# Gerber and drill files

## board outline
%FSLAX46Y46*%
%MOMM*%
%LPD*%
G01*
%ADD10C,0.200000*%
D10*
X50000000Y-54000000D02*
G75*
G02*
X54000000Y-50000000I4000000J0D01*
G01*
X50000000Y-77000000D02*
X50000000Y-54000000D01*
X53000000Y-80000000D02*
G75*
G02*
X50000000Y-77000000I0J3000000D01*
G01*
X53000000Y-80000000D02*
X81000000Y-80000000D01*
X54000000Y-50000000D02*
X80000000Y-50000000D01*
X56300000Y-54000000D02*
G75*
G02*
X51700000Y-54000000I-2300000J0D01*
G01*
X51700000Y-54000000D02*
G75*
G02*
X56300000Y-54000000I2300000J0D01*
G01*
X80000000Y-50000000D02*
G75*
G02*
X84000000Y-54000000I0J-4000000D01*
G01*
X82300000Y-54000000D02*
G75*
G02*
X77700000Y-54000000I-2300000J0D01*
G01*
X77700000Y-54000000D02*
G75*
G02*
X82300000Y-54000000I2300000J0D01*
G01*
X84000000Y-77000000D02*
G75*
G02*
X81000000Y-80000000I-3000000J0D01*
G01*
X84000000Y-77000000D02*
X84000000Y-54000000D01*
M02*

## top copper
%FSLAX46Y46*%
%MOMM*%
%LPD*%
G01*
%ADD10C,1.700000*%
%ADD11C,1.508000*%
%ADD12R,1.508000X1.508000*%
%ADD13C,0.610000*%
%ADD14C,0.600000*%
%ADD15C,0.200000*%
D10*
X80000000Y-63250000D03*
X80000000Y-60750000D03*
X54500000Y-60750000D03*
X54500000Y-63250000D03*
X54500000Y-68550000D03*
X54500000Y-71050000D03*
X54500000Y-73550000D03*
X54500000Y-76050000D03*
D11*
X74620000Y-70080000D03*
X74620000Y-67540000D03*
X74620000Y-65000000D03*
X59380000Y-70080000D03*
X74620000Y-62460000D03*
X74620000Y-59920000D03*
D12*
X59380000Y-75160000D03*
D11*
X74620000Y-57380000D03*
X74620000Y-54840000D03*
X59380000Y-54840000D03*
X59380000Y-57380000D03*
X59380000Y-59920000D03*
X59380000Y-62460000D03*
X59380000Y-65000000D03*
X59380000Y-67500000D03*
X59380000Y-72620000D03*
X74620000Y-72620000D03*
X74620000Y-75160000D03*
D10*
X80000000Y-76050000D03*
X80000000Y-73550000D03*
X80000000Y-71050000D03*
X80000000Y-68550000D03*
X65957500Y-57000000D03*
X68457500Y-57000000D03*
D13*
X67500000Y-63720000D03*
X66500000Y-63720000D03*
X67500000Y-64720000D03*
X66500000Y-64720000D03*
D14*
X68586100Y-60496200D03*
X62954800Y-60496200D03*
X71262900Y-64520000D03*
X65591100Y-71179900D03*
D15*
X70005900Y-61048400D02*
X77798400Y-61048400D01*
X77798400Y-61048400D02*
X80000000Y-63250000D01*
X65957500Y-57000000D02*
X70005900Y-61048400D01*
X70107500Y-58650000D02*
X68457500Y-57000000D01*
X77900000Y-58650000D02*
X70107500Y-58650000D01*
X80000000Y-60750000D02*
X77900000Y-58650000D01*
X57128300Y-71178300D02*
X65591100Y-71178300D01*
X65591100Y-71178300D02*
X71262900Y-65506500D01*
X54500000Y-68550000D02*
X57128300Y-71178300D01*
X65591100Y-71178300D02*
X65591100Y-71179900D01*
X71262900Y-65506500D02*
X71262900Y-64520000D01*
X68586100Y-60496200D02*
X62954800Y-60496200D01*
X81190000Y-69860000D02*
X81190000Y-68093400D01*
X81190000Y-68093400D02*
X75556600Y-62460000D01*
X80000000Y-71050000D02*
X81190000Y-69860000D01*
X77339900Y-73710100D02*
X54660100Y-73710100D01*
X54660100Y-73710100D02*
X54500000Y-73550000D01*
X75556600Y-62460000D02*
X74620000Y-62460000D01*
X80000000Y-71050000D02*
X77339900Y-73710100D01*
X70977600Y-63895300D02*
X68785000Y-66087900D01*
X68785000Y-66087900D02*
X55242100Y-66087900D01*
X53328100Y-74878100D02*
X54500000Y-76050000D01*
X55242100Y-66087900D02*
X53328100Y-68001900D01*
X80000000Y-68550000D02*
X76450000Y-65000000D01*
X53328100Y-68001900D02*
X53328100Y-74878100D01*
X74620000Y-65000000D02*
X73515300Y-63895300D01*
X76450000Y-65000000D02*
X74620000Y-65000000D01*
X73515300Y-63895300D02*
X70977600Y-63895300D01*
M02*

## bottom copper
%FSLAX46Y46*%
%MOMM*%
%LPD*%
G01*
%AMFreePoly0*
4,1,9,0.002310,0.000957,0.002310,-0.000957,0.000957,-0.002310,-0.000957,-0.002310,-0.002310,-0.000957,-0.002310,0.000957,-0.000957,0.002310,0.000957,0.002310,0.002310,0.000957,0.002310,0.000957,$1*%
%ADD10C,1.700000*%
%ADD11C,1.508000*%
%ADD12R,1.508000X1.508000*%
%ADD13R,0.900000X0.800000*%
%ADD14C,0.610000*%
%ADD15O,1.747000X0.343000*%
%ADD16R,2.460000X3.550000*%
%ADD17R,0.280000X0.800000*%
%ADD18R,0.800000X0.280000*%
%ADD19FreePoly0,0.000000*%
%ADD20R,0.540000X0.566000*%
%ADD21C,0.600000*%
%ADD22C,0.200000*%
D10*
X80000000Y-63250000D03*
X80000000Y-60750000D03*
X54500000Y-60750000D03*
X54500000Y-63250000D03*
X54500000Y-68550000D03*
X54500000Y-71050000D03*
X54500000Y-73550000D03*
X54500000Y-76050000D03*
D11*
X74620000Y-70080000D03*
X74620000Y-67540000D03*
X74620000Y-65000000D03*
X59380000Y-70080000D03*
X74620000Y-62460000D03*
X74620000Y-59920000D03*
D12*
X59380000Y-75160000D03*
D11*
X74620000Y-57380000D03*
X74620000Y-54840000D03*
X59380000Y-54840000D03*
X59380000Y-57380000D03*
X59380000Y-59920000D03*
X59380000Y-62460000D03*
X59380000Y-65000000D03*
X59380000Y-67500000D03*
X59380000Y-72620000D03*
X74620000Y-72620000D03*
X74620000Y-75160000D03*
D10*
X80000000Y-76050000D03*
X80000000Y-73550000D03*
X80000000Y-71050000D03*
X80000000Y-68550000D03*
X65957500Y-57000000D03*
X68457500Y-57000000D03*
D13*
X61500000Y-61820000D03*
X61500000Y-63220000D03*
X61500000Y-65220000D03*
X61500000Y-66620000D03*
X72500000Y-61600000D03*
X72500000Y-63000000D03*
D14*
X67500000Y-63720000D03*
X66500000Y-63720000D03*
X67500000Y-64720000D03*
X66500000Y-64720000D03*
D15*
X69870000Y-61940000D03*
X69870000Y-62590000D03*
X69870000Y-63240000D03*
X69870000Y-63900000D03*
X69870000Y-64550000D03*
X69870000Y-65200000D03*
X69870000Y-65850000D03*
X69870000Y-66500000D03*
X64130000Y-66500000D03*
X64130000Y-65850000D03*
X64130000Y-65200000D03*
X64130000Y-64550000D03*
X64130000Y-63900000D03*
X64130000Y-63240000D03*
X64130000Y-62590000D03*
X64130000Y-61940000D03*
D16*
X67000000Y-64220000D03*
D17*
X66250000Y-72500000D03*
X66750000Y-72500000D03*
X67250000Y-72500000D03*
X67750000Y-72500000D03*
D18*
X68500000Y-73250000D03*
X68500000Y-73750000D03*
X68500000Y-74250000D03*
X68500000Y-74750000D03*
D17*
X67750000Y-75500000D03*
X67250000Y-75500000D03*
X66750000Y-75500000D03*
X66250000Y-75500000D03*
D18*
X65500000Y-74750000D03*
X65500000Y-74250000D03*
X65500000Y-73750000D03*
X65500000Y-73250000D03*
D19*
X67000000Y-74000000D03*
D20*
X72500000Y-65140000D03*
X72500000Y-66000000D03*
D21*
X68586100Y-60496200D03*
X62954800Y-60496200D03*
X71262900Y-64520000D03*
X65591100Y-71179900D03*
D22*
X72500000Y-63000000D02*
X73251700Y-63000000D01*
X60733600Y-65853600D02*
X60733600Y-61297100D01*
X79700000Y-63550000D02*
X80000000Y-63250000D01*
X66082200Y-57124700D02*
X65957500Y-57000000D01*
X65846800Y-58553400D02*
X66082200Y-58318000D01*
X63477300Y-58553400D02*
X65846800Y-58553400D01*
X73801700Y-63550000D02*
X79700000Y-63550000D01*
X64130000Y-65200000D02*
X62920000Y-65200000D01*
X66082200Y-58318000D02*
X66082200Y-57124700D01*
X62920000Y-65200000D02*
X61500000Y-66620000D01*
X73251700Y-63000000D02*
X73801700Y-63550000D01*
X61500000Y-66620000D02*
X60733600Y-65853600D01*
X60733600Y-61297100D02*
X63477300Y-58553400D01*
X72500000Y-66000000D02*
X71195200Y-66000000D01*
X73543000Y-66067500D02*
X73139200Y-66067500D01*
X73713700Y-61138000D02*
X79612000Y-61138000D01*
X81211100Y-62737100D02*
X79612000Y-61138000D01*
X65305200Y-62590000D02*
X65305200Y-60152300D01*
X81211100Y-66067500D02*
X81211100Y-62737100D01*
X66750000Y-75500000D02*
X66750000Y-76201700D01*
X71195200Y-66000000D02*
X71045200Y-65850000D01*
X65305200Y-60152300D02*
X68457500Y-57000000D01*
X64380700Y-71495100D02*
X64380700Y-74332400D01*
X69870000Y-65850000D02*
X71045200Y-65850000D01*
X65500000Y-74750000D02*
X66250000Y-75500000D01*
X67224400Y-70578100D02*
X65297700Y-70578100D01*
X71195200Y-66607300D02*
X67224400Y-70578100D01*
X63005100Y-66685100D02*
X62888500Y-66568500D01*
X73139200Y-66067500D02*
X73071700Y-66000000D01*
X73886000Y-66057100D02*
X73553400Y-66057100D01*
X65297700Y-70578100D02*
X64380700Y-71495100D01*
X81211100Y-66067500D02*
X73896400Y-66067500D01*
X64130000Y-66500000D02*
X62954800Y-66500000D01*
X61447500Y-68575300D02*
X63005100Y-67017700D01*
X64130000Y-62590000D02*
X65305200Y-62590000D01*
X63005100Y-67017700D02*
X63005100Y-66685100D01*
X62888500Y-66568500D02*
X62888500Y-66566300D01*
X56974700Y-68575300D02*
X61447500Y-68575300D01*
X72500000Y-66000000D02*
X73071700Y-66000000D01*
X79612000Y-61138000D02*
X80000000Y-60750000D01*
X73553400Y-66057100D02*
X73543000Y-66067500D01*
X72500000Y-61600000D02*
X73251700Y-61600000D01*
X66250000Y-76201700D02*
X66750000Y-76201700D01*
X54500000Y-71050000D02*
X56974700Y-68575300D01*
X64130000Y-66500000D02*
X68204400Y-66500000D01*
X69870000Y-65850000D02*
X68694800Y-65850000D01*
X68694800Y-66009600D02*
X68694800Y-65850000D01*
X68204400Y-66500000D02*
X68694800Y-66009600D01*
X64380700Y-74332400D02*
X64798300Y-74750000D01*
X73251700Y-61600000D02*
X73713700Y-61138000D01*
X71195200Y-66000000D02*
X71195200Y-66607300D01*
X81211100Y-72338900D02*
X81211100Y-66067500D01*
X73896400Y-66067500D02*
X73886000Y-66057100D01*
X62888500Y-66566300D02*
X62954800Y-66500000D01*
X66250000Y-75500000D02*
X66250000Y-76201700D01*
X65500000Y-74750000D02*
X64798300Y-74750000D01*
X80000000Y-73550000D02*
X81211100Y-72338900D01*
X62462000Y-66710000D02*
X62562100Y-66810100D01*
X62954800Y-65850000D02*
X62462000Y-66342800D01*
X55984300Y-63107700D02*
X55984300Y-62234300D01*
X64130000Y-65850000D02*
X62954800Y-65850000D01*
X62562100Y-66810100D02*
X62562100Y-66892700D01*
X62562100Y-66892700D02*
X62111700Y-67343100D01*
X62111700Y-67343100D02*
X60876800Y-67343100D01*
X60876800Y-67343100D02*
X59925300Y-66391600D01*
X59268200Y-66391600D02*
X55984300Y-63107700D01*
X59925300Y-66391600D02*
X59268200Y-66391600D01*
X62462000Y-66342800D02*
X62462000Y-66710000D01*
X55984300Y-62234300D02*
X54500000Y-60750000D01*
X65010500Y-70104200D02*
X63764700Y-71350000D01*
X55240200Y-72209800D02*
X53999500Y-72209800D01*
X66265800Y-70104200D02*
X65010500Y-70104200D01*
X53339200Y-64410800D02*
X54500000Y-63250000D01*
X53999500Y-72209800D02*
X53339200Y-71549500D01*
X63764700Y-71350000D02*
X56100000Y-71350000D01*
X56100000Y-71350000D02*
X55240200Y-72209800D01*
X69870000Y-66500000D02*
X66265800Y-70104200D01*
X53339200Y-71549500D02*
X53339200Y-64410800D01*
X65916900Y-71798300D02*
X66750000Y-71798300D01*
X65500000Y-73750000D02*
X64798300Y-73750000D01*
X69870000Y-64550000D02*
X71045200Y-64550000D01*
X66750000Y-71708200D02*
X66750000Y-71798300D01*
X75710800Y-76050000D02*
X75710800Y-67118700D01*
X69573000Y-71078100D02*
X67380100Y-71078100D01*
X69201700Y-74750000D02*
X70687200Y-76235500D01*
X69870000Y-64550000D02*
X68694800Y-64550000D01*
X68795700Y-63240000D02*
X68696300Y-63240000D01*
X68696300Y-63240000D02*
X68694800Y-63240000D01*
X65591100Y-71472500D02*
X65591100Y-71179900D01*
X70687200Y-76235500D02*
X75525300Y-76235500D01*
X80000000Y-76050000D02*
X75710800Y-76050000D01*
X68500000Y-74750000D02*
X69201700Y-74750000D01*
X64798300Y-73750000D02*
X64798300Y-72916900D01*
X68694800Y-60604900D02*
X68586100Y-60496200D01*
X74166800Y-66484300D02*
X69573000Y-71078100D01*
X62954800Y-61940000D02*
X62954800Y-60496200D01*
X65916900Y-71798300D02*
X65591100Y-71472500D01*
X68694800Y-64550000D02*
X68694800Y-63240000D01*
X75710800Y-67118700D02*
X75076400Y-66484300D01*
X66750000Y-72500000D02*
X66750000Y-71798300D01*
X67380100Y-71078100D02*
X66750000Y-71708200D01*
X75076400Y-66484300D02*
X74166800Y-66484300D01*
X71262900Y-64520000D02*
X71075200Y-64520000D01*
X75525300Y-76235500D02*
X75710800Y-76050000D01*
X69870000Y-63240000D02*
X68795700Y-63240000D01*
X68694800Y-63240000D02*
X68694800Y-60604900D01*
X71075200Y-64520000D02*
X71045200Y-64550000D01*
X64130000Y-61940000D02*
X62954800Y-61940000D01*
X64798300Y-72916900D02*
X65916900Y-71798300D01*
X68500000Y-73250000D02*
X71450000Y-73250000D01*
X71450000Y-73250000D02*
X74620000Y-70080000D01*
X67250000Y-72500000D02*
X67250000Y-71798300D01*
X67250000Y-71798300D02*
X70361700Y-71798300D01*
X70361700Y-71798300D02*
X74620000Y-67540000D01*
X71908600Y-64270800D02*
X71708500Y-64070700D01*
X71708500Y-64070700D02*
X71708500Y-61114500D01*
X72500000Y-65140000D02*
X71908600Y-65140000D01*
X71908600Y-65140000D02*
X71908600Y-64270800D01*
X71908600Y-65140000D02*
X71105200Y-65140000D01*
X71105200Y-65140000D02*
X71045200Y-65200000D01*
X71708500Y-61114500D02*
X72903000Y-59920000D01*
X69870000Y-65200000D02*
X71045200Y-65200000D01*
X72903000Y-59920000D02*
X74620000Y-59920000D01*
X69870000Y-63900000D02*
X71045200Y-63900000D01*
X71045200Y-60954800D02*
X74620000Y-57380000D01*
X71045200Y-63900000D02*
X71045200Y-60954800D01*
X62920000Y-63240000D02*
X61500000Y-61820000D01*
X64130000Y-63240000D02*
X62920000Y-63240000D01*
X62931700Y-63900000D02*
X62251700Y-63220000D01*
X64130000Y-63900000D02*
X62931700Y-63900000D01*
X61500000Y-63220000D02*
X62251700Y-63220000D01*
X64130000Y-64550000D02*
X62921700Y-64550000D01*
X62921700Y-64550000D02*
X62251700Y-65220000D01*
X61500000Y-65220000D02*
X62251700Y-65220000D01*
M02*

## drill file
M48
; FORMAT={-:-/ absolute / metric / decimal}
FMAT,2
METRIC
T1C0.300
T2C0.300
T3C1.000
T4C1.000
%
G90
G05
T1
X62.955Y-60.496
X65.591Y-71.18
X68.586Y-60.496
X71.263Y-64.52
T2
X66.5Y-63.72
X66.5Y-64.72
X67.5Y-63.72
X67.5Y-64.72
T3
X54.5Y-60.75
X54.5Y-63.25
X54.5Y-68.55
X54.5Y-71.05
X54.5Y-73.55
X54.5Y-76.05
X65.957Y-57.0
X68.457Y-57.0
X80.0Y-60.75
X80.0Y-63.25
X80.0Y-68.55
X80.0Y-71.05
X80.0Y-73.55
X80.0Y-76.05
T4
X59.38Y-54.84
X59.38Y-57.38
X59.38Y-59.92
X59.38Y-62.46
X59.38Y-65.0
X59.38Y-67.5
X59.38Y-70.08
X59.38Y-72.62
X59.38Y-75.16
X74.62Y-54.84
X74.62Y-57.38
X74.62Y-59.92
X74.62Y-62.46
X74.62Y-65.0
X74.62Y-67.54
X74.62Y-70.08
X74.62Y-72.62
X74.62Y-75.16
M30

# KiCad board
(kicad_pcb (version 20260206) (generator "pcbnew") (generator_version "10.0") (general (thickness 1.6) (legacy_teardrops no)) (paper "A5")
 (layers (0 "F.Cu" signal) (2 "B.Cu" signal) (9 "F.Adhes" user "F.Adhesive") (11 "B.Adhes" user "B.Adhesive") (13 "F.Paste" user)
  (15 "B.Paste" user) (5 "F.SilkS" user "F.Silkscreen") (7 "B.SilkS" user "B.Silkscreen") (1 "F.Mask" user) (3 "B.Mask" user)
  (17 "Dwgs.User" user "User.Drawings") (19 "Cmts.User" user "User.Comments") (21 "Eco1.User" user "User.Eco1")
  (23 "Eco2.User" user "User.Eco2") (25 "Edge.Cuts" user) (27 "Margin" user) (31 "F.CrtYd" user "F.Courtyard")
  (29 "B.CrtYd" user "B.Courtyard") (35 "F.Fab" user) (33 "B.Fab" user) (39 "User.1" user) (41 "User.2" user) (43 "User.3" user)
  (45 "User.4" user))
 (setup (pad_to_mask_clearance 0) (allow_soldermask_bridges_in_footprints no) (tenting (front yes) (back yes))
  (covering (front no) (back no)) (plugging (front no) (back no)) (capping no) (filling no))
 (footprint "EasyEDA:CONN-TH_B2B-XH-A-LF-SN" (layer "F.Cu") (at 80 62 -90)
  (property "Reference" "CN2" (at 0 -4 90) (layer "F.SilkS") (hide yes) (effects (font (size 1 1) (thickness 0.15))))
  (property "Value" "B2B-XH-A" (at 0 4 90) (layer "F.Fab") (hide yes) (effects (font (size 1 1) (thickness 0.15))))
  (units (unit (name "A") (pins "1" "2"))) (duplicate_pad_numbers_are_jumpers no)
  (pad "1" thru_hole circle (at 1.25 0 90) (size 1.7 1.7) (drill 0.999998) (layers "*.Cu" "*.Mask") (remove_unused_layers no)
   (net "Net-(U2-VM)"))
  (pad "2" thru_hole circle (at -1.25 0 90) (size 1.7 1.7) (drill 0.999998) (layers "*.Cu" "*.Mask") (remove_unused_layers no)
   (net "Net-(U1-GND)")))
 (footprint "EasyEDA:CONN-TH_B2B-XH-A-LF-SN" (layer "F.Cu") (at 54.5 62 90)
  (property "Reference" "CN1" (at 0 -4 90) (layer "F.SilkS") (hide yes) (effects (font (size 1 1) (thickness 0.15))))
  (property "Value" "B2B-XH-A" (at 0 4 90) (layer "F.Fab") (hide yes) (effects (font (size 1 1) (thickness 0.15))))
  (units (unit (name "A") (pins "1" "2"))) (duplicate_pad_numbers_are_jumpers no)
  (pad "1" thru_hole circle (at 1.25 0 270) (size 1.7 1.7) (drill 0.999998) (layers "*.Cu" "*.Mask") (remove_unused_layers no)
   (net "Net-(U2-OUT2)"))
  (pad "2" thru_hole circle (at -1.25 0 270) (size 1.7 1.7) (drill 0.999998) (layers "*.Cu" "*.Mask") (remove_unused_layers no)
   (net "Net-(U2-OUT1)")))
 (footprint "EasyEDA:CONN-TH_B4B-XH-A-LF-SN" (layer "F.Cu") (at 54.5 72.3 90)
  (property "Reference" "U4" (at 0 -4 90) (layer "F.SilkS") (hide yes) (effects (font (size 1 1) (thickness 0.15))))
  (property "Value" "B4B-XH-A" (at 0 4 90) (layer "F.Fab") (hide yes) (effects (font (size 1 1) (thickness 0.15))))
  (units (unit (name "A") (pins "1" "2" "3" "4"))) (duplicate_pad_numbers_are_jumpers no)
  (pad "1" thru_hole circle (at 3.75 0 90) (size 1.7 1.7) (drill 0.999998) (layers "*.Cu" "*.Mask") (remove_unused_layers no)
   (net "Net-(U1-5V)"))
  (pad "2" thru_hole circle (at 1.25 0 90) (size 1.7 1.7) (drill 0.999998) (layers "*.Cu" "*.Mask") (remove_unused_layers no)
   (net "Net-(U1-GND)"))
  (pad "3" thru_hole circle (at -1.25 0 90) (size 1.7 1.7) (drill 0.999998) (layers "*.Cu" "*.Mask") (remove_unused_layers no)
   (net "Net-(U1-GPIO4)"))
  (pad "4" thru_hole circle (at -3.75 0 90) (size 1.7 1.7) (drill 0.999998) (layers "*.Cu" "*.Mask") (remove_unused_layers no)
   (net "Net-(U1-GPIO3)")))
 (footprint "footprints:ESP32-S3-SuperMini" (layer "F.Cu") (at 67 65 180)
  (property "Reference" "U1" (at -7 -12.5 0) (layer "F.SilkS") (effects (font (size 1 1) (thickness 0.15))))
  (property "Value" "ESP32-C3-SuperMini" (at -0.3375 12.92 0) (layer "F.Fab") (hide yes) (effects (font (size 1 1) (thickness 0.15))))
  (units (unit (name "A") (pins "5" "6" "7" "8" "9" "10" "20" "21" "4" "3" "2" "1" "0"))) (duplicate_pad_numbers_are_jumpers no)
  (pad "1" thru_hole circle (at -7.62 -5.08 180) (size 1.508 1.508) (drill 1) (layers "*.Cu" "*.Mask") (remove_unused_layers no)
   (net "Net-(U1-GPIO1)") (solder_mask_margin 0.102))
  (pad "2" thru_hole circle (at -7.62 -2.54 180) (size 1.508 1.508) (drill 1) (layers "*.Cu" "*.Mask") (remove_unused_layers no)
   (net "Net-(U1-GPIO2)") (solder_mask_margin 0.102))
  (pad "3" thru_hole circle (at -7.62 0 180) (size 1.508 1.508) (drill 1) (layers "*.Cu" "*.Mask") (remove_unused_layers no)
   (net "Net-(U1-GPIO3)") (solder_mask_margin 0.102))
  (pad "3V3" thru_hole circle (at 7.62 -5.08 180) (size 1.508 1.508) (drill 1) (layers "*.Cu" "*.Mask") (remove_unused_layers no)
   (solder_mask_margin 0.102))
  (pad "4" thru_hole circle (at -7.62 2.54 180) (size 1.508 1.508) (drill 1) (layers "*.Cu" "*.Mask") (remove_unused_layers no)
   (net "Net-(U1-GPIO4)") (solder_mask_margin 0.102))
  (pad "5" thru_hole circle (at -7.62 5.08 180) (size 1.508 1.508) (drill 1) (layers "*.Cu" "*.Mask") (remove_unused_layers no)
   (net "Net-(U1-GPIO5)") (solder_mask_margin 0.102))
  (pad "5V" thru_hole rect (at 7.62 -10.16 180) (size 1.508 1.508) (drill 1) (layers "*.Cu" "*.Mask") (remove_unused_layers no)
   (solder_mask_margin 0.102))
  (pad "6" thru_hole circle (at -7.62 7.62 180) (size 1.508 1.508) (drill 1) (layers "*.Cu" "*.Mask") (remove_unused_layers no)
   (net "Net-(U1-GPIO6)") (solder_mask_margin 0.102))
  (pad "7" thru_hole circle (at -7.62 10.16 180) (size 1.508 1.508) (drill 1) (layers "*.Cu" "*.Mask") (remove_unused_layers no)
   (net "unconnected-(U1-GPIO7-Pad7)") (solder_mask_margin 0.102))
  (pad "8" thru_hole circle (at 7.62 10.16 180) (size 1.508 1.508) (drill 1) (layers "*.Cu" "*.Mask") (remove_unused_layers no)
   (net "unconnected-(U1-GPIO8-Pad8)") (solder_mask_margin 0.102))
  (pad "9" thru_hole circle (at 7.62 7.62 180) (size 1.508 1.508) (drill 1) (layers "*.Cu" "*.Mask") (remove_unused_layers no)
   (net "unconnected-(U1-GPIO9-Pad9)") (solder_mask_margin 0.102))
  (pad "10" thru_hole circle (at 7.62 5.08 180) (size 1.508 1.508) (drill 1) (layers "*.Cu" "*.Mask") (remove_unused_layers no)
   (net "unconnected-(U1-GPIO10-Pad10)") (solder_mask_margin 0.102))
  (pad "11" thru_hole circle (at 7.62 2.54 180) (size 1.508 1.508) (drill 1) (layers "*.Cu" "*.Mask") (remove_unused_layers no)
   (solder_mask_margin 0.102))
  (pad "12" thru_hole circle (at 7.62 0 180) (size 1.508 1.508) (drill 1) (layers "*.Cu" "*.Mask") (remove_unused_layers no)
   (solder_mask_margin 0.102))
  (pad "13" thru_hole circle (at 7.62 -2.5 180) (size 1.508 1.508) (drill 1) (layers "*.Cu" "*.Mask") (remove_unused_layers no)
   (solder_mask_margin 0.102))
  (pad "GND" thru_hole circle (at 7.62 -7.62 180) (size 1.508 1.508) (drill 1) (layers "*.Cu" "*.Mask") (remove_unused_layers no)
   (solder_mask_margin 0.102))
  (pad "RX" thru_hole circle (at -7.62 -7.62 180) (size 1.508 1.508) (drill 1) (layers "*.Cu" "*.Mask") (remove_unused_layers no)
   (solder_mask_margin 0.102))
  (pad "TX" thru_hole circle (at -7.62 -10.16 180) (size 1.508 1.508) (drill 1) (layers "*.Cu" "*.Mask") (remove_unused_layers no)
   (solder_mask_margin 0.102)))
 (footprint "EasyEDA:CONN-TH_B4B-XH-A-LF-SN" (layer "F.Cu") (at 80 72.3 -90)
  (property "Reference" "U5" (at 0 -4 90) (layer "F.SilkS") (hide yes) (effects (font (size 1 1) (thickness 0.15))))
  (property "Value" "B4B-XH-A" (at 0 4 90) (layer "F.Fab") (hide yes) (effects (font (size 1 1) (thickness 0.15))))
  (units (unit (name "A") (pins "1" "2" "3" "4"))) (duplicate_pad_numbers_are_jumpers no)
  (pad "1" thru_hole circle (at 3.75 0 270) (size 1.7 1.7) (drill 0.999998) (layers "*.Cu" "*.Mask") (remove_unused_layers no)
   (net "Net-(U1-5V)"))
  (pad "2" thru_hole circle (at 1.25 0 270) (size 1.7 1.7) (drill 0.999998) (layers "*.Cu" "*.Mask") (remove_unused_layers no)
   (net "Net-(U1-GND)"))
  (pad "3" thru_hole circle (at -1.25 0 270) (size 1.7 1.7) (drill 0.999998) (layers "*.Cu" "*.Mask") (remove_unused_layers no)
   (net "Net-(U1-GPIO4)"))
  (pad "4" thru_hole circle (at -3.75 0 270) (size 1.7 1.7) (drill 0.999998) (layers "*.Cu" "*.Mask") (remove_unused_layers no)
   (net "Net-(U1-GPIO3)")))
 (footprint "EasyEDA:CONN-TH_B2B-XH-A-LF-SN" (layer "B.Cu") (at 67.2075 57 180)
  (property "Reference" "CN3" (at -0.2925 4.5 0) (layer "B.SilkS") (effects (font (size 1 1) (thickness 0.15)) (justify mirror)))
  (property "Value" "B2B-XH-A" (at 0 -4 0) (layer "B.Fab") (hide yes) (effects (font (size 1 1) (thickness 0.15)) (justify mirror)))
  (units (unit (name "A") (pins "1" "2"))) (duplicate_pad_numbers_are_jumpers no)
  (pad "1" thru_hole circle (at 1.25 0) (size 1.7 1.7) (drill 0.999998) (layers "*.Cu" "*.Mask") (remove_unused_layers no)
   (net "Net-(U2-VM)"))
  (pad "2" thru_hole circle (at -1.25 0) (size 1.7 1.7) (drill 0.999998) (layers "*.Cu" "*.Mask") (remove_unused_layers no)
   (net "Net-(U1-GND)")))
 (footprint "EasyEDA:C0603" (layer "B.Cu") (at 61.5 62.52 -90)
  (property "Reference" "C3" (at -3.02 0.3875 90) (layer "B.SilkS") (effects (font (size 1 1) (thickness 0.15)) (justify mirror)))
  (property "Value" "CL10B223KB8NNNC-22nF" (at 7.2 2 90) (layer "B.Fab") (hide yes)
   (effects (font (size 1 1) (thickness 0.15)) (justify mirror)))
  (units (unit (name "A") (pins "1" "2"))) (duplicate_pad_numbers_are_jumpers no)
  (pad "1" smd rect (at -0.7 0 270) (size 0.8 0.9) (layers "B.Cu" "B.Mask" "B.Paste") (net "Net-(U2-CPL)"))
  (pad "2" smd rect (at 0.7 0 270) (size 0.8 0.9) (layers "B.Cu" "B.Mask" "B.Paste") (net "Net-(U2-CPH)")))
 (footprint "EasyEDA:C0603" (layer "B.Cu") (at 61.5 65.92 -90)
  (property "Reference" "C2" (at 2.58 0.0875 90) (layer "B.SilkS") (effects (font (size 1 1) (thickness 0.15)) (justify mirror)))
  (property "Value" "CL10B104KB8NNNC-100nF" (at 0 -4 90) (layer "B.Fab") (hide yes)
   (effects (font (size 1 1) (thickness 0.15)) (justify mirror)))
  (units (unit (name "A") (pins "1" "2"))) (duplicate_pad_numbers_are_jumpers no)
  (pad "1" smd rect (at -0.7 0 270) (size 0.8 0.9) (layers "B.Cu" "B.Mask" "B.Paste") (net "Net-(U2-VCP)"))
  (pad "2" smd rect (at 0.7 0 270) (size 0.8 0.9) (layers "B.Cu" "B.Mask" "B.Paste") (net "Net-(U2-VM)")))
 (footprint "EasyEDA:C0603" (layer "B.Cu") (at 72.5 62.3 -90)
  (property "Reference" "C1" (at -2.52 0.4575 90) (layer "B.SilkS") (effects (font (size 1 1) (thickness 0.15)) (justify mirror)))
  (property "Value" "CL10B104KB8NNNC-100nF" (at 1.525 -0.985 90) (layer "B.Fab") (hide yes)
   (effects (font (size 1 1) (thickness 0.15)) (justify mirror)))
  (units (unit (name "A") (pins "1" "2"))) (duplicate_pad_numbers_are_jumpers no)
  (pad "1" smd rect (at -0.7 0 270) (size 0.8 0.9) (layers "B.Cu" "B.Mask" "B.Paste") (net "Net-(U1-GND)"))
  (pad "2" smd rect (at 0.7 0 270) (size 0.8 0.9) (layers "B.Cu" "B.Mask" "B.Paste") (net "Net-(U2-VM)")))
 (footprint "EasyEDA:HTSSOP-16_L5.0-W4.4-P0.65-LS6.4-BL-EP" (layer "B.Cu") (at 67 64.22 -90)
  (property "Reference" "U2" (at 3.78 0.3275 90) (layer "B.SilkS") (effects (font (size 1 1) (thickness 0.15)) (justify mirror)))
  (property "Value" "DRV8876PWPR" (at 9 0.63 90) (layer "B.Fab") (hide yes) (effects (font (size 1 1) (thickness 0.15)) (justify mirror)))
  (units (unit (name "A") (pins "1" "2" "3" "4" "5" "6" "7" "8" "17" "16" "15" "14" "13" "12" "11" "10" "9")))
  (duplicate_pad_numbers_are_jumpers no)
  (pad "" thru_hole circle (at -0.5 -0.5 270) (size 0.61 0.61) (drill 0.3) (layers "*.Cu" "*.Paste" "*.Mask") (remove_unused_layers no))
  (pad "" thru_hole circle (at -0.5 0.5 270) (size 0.61 0.61) (drill 0.3) (layers "*.Cu" "*.Paste" "*.Mask") (remove_unused_layers no))
  (pad "" thru_hole circle (at 0.5 -0.5 270) (size 0.61 0.61) (drill 0.3) (layers "*.Cu" "*.Paste" "*.Mask") (remove_unused_layers no))
  (pad "" thru_hole circle (at 0.5 0.5 270) (size 0.61 0.61) (drill 0.3) (layers "*.Cu" "*.Paste" "*.Mask") (remove_unused_layers no))
  (pad "1" smd oval (at -2.28 -2.87 270) (size 0.343 1.747) (layers "B.Cu" "B.Mask" "B.Paste") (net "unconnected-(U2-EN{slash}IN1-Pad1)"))
  (pad "2" smd oval (at -1.63 -2.87 270) (size 0.343 1.747) (layers "B.Cu" "B.Mask" "B.Paste") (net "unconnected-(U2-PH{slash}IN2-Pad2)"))
  (pad "3" smd oval (at -0.98 -2.87 270) (size 0.343 1.747) (layers "B.Cu" "B.Mask" "B.Paste") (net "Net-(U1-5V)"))
  (pad "4" smd oval (at -0.32 -2.87 270) (size 0.343 1.747) (layers "B.Cu" "B.Mask" "B.Paste") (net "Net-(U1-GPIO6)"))
  (pad "5" smd oval (at 0.33 -2.87 270) (size 0.343 1.747) (layers "B.Cu" "B.Mask" "B.Paste") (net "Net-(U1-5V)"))
  (pad "6" smd oval (at 0.98 -2.87 270) (size 0.343 1.747) (layers "B.Cu" "B.Mask" "B.Paste") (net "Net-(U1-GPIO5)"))
  (pad "7" smd oval (at 1.63 -2.87 270) (size 0.343 1.747) (layers "B.Cu" "B.Mask" "B.Paste") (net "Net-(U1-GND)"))
  (pad "8" smd oval (at 2.28 -2.87 270) (size 0.343 1.747) (layers "B.Cu" "B.Mask" "B.Paste") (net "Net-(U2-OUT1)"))
  (pad "9" smd oval (at 2.28 2.87 270) (size 0.343 1.747) (layers "B.Cu" "B.Mask" "B.Paste") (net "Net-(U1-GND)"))
  (pad "10" smd oval (at 1.63 2.87 270) (size 0.343 1.747) (layers "B.Cu" "B.Mask" "B.Paste") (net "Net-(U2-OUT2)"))
  (pad "11" smd oval (at 0.98 2.87 270) (size 0.343 1.747) (layers "B.Cu" "B.Mask" "B.Paste") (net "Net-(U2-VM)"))
  (pad "12" smd oval (at 0.33 2.87 270) (size 0.343 1.747) (layers "B.Cu" "B.Mask" "B.Paste") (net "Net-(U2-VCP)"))
  (pad "13" smd oval (at -0.32 2.87 270) (size 0.343 1.747) (layers "B.Cu" "B.Mask" "B.Paste") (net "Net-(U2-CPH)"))
  (pad "14" smd oval (at -0.98 2.87 270) (size 0.343 1.747) (layers "B.Cu" "B.Mask" "B.Paste") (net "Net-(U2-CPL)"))
  (pad "15" smd oval (at -1.63 2.87 270) (size 0.343 1.747) (layers "B.Cu" "B.Mask" "B.Paste") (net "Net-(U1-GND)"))
  (pad "16" smd oval (at -2.28 2.87 270) (size 0.343 1.747) (layers "B.Cu" "B.Mask" "B.Paste") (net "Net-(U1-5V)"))
  (pad "17" smd rect (at 0 0 270) (size 3.55 2.46) (layers "B.Cu" "B.Mask" "B.Paste") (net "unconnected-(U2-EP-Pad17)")))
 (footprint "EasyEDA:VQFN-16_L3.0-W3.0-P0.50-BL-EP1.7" (layer "B.Cu") (at 67 74)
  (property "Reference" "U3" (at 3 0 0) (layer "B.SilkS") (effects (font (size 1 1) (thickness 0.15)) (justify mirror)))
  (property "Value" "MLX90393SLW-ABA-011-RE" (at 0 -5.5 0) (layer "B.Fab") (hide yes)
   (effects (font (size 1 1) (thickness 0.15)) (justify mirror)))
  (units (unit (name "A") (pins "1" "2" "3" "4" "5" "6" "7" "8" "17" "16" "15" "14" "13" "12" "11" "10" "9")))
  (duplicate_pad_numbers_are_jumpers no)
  (pad "1" smd rect (at -0.75 -1.5) (size 0.28 0.8) (layers "B.Cu" "B.Mask" "B.Paste") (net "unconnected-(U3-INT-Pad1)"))
  (pad "2" smd rect (at -0.25 -1.5) (size 0.28 0.8) (layers "B.Cu" "B.Mask" "B.Paste") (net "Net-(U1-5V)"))
  (pad "3" smd rect (at 0.25 -1.5) (size 0.28 0.8) (layers "B.Cu" "B.Mask" "B.Paste") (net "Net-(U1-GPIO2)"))
  (pad "4" smd rect (at 0.75 -1.5) (size 0.28 0.8) (layers "B.Cu" "B.Mask" "B.Paste") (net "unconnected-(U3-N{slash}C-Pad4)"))
  (pad "5" smd rect (at 1.5 -0.75) (size 0.8 0.28) (layers "B.Cu" "B.Mask" "B.Paste") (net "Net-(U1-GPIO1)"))
  (pad "6" smd rect (at 1.5 -0.25) (size 0.8 0.28) (layers "B.Cu" "B.Mask" "B.Paste") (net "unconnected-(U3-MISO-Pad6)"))
  (pad "7" smd rect (at 1.5 0.25) (size 0.8 0.28) (layers "B.Cu" "B.Mask" "B.Paste") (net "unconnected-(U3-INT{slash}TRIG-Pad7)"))
  (pad "8" smd rect (at 1.5 0.75) (size 0.8 0.28) (layers "B.Cu" "B.Mask" "B.Paste") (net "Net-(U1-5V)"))
  (pad "9" smd rect (at 0.75 1.5) (size 0.28 0.8) (layers "B.Cu" "B.Mask" "B.Paste") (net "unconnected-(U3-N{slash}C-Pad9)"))
  (pad "10" smd rect (at 0.25 1.5) (size 0.28 0.8) (layers "B.Cu" "B.Mask" "B.Paste") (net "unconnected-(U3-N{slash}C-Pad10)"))
  (pad "11" smd rect (at -0.25 1.5) (size 0.28 0.8) (layers "B.Cu" "B.Mask" "B.Paste") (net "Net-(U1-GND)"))
  (pad "12" smd rect (at -0.75 1.5) (size 0.28 0.8) (layers "B.Cu" "B.Mask" "B.Paste") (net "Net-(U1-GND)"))
  (pad "13" smd rect (at -1.5 0.75) (size 0.8 0.28) (layers "B.Cu" "B.Mask" "B.Paste") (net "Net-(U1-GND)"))
  (pad "14" smd rect (at -1.5 0.25) (size 0.8 0.28) (layers "B.Cu" "B.Mask" "B.Paste") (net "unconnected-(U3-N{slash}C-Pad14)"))
  (pad "15" smd rect (at -1.5 -0.25) (size 0.8 0.28) (layers "B.Cu" "B.Mask" "B.Paste") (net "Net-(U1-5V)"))
  (pad "16" smd rect (at -1.5 -0.75) (size 0.8 0.28) (layers "B.Cu" "B.Mask" "B.Paste") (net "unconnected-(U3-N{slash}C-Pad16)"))
  (pad "17" smd custom (at 0 0) (size 0.005 0.005) (layers "B.Cu" "B.Mask" "B.Paste") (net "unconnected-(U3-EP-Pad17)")
   (thermal_bridge_angle 90) (options (clearance outline) (anchor circle)) (primitives)))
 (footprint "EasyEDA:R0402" (layer "B.Cu") (at 72.5 65.57 -90)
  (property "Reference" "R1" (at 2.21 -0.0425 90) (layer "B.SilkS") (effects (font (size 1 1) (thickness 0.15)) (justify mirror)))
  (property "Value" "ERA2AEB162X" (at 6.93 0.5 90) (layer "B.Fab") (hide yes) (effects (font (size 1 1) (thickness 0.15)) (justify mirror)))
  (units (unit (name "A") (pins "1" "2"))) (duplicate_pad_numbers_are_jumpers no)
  (pad "1" smd rect (at -0.43 0 270) (size 0.566 0.54) (layers "B.Cu" "B.Mask" "B.Paste") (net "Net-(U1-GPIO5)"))
  (pad "2" smd rect (at 0.43 0 270) (size 0.566 0.54) (layers "B.Cu" "B.Mask" "B.Paste") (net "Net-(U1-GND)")))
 (gr_arc (start 50 54) (mid 51.171573 51.171573) (end 54 50) (stroke (width 0.2) (type solid)) (layer "Edge.Cuts"))
 (gr_line (start 50 77) (end 50 54) (stroke (width 0.2) (type solid)) (layer "Edge.Cuts"))
 (gr_arc (start 53 80) (mid 50.87868 79.12132) (end 50 77) (stroke (width 0.2) (type solid)) (layer "Edge.Cuts"))
 (gr_line (start 53 80) (end 81 80) (stroke (width 0.2) (type default)) (layer "Edge.Cuts"))
 (gr_line (start 54 50) (end 80 50) (stroke (width 0.2) (type default)) (layer "Edge.Cuts"))
 (gr_circle (center 54 54) (end 56.3 54) (stroke (width 0.2) (type solid)) (fill no) (layer "Edge.Cuts"))
 (gr_arc (start 80 50) (mid 82.828427 51.171573) (end 84 54) (stroke (width 0.2) (type solid)) (layer "Edge.Cuts"))
 (gr_circle (center 80 54) (end 82.3 54) (stroke (width 0.2) (type default)) (fill no) (layer "Edge.Cuts"))
 (gr_arc (start 84 77) (mid 83.12132 79.12132) (end 81 80) (stroke (width 0.2) (type solid)) (layer "Edge.Cuts"))
 (gr_line (start 84 77) (end 84 54) (stroke (width 0.2) (type solid)) (layer "Edge.Cuts"))
 (segment (start 70.0059 61.0484) (end 77.7984 61.0484) (width 0.2) (layer "F.Cu") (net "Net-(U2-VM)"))
 (segment (start 77.7984 61.0484) (end 80 63.25) (width 0.2) (layer "F.Cu") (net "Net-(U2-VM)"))
 (segment (start 65.9575 57) (end 70.0059 61.0484) (width 0.2) (layer "F.Cu") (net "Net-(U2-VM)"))
 (segment (start 72.5 63) (end 73.2517 63) (width 0.2) (layer "B.Cu") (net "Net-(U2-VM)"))
 (segment (start 60.7336 65.8536) (end 60.7336 61.2971) (width 0.2) (layer "B.Cu") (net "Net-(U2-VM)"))
 (segment (start 79.7 63.55) (end 80 63.25) (width 0.2) (layer "B.Cu") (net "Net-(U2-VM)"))
 (segment (start 66.0822 57.1247) (end 65.9575 57) (width 0.2) (layer "B.Cu") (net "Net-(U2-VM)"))
 (segment (start 65.8468 58.5534) (end 66.0822 58.318) (width 0.2) (layer "B.Cu") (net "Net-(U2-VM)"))
 (segment (start 63.4773 58.5534) (end 65.8468 58.5534) (width 0.2) (layer "B.Cu") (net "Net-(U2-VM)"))
 (segment (start 73.8017 63.55) (end 79.7 63.55) (width 0.2) (layer "B.Cu") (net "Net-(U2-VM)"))
 (segment (start 64.13 65.2) (end 62.92 65.2) (width 0.2) (layer "B.Cu") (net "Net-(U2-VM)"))
 (segment (start 66.0822 58.318) (end 66.0822 57.1247) (width 0.2) (layer "B.Cu") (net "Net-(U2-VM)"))
 (segment (start 62.92 65.2) (end 61.5 66.62) (width 0.2) (layer "B.Cu") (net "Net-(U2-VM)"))
 (segment (start 73.2517 63) (end 73.8017 63.55) (width 0.2) (layer "B.Cu") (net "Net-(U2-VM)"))
 (segment (start 61.5 66.62) (end 60.7336 65.8536) (width 0.2) (layer "B.Cu") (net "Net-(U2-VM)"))
 (segment (start 60.7336 61.2971) (end 63.4773 58.5534) (width 0.2) (layer "B.Cu") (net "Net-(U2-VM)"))
 (segment (start 70.1075 58.65) (end 68.4575 57) (width 0.2) (layer "F.Cu") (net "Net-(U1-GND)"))
 (segment (start 77.9 58.65) (end 70.1075 58.65) (width 0.2) (layer "F.Cu") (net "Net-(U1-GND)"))
 (segment (start 80 60.75) (end 77.9 58.65) (width 0.2) (layer "F.Cu") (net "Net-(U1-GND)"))
 (segment (start 72.5 66) (end 71.1952 66) (width 0.2) (layer "B.Cu") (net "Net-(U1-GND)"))
 (segment (start 73.543 66.0675) (end 73.1392 66.0675) (width 0.2) (layer "B.Cu") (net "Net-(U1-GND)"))
 (segment (start 73.7137 61.138) (end 79.612 61.138) (width 0.2) (layer "B.Cu") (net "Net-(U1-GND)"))
 (segment (start 81.2111 62.7371) (end 79.612 61.138) (width 0.2) (layer "B.Cu") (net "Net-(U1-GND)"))
 (segment (start 65.3052 62.59) (end 65.3052 60.1523) (width 0.2) (layer "B.Cu") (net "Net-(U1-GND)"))
 (segment (start 81.2111 66.0675) (end 81.2111 62.7371) (width 0.2) (layer "B.Cu") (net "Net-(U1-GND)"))
 (segment (start 66.75 75.5) (end 66.75 76.2017) (width 0.2) (layer "B.Cu") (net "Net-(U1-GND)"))
 (segment (start 71.1952 66) (end 71.0452 65.85) (width 0.2) (layer "B.Cu") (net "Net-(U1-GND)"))
 (segment (start 65.3052 60.1523) (end 68.4575 57) (width 0.2) (layer "B.Cu") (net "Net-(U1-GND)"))
 (segment (start 64.3807 71.4951) (end 64.3807 74.3324) (width 0.2) (layer "B.Cu") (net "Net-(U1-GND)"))
 (segment (start 69.87 65.85) (end 71.0452 65.85) (width 0.2) (layer "B.Cu") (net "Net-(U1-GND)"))
 (segment (start 65.5 74.75) (end 66.25 75.5) (width 0.2) (layer "B.Cu") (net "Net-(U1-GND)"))
 (segment (start 67.2244 70.5781) (end 65.2977 70.5781) (width 0.2) (layer "B.Cu") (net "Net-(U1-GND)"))
 (segment (start 71.1952 66.6073) (end 67.2244 70.5781) (width 0.2) (layer "B.Cu") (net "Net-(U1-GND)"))
 (segment (start 63.0051 66.6851) (end 62.8885 66.5685) (width 0.2) (layer "B.Cu") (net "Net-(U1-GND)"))
 (segment (start 73.1392 66.0675) (end 73.0717 66) (width 0.2) (layer "B.Cu") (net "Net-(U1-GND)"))
 (segment (start 73.886 66.0571) (end 73.5534 66.0571) (width 0.2) (layer "B.Cu") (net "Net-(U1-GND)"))
 (segment (start 65.2977 70.5781) (end 64.3807 71.4951) (width 0.2) (layer "B.Cu") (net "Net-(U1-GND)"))
 (segment (start 81.2111 66.0675) (end 73.8964 66.0675) (width 0.2) (layer "B.Cu") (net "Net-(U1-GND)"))
 (segment (start 64.13 66.5) (end 62.9548 66.5) (width 0.2) (layer "B.Cu") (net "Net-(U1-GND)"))
 (segment (start 61.4475 68.5753) (end 63.0051 67.0177) (width 0.2) (layer "B.Cu") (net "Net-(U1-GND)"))
 (segment (start 64.13 62.59) (end 65.3052 62.59) (width 0.2) (layer "B.Cu") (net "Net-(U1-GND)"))
 (segment (start 63.0051 67.0177) (end 63.0051 66.6851) (width 0.2) (layer "B.Cu") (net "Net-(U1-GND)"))
 (segment (start 62.8885 66.5685) (end 62.8885 66.5663) (width 0.2) (layer "B.Cu") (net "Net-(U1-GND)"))
 (segment (start 56.9747 68.5753) (end 61.4475 68.5753) (width 0.2) (layer "B.Cu") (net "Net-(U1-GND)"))
 (segment (start 72.5 66) (end 73.0717 66) (width 0.2) (layer "B.Cu") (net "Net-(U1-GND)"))
 (segment (start 79.612 61.138) (end 80 60.75) (width 0.2) (layer "B.Cu") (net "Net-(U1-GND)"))
 (segment (start 73.5534 66.0571) (end 73.543 66.0675) (width 0.2) (layer "B.Cu") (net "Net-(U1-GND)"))
 (segment (start 72.5 61.6) (end 73.2517 61.6) (width 0.2) (layer "B.Cu") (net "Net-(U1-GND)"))
 (segment (start 66.25 76.2017) (end 66.75 76.2017) (width 0.2) (layer "B.Cu") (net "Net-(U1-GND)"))
 (segment (start 54.5 71.05) (end 56.9747 68.5753) (width 0.2) (layer "B.Cu") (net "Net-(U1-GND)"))
 (segment (start 64.13 66.5) (end 68.2044 66.5) (width 0.2) (layer "B.Cu") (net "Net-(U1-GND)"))
 (segment (start 69.87 65.85) (end 68.6948 65.85) (width 0.2) (layer "B.Cu") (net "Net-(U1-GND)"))
 (segment (start 68.6948 66.0096) (end 68.6948 65.85) (width 0.2) (layer "B.Cu") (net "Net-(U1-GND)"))
 (segment (start 68.2044 66.5) (end 68.6948 66.0096) (width 0.2) (layer "B.Cu") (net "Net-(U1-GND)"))
 (segment (start 64.3807 74.3324) (end 64.7983 74.75) (width 0.2) (layer "B.Cu") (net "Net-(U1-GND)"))
 (segment (start 73.2517 61.6) (end 73.7137 61.138) (width 0.2) (layer "B.Cu") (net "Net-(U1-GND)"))
 (segment (start 71.1952 66) (end 71.1952 66.6073) (width 0.2) (layer "B.Cu") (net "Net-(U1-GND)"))
 (segment (start 81.2111 72.3389) (end 81.2111 66.0675) (width 0.2) (layer "B.Cu") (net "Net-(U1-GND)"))
 (segment (start 73.8964 66.0675) (end 73.886 66.0571) (width 0.2) (layer "B.Cu") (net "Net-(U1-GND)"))
 (segment (start 62.8885 66.5663) (end 62.9548 66.5) (width 0.2) (layer "B.Cu") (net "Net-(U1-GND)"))
 (segment (start 66.25 75.5) (end 66.25 76.2017) (width 0.2) (layer "B.Cu") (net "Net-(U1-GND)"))
 (segment (start 65.5 74.75) (end 64.7983 74.75) (width 0.2) (layer "B.Cu") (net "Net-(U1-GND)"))
 (segment (start 80 73.55) (end 81.2111 72.3389) (width 0.2) (layer "B.Cu") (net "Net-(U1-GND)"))
 (segment (start 62.462 66.71) (end 62.5621 66.8101) (width 0.2) (layer "B.Cu") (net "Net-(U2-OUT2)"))
 (segment (start 62.9548 65.85) (end 62.462 66.3428) (width 0.2) (layer "B.Cu") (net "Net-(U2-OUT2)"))
 (segment (start 55.9843 63.1077) (end 55.9843 62.2343) (width 0.2) (layer "B.Cu") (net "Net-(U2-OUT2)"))
 (segment (start 64.13 65.85) (end 62.9548 65.85) (width 0.2) (layer "B.Cu") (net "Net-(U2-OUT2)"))
 (segment (start 62.5621 66.8101) (end 62.5621 66.8927) (width 0.2) (layer "B.Cu") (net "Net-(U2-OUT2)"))
 (segment (start 62.5621 66.8927) (end 62.1117 67.3431) (width 0.2) (layer "B.Cu") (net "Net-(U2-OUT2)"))
 (segment (start 62.1117 67.3431) (end 60.8768 67.3431) (width 0.2) (layer "B.Cu") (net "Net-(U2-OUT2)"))
 (segment (start 60.8768 67.3431) (end 59.9253 66.3916) (width 0.2) (layer "B.Cu") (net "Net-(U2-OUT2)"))
 (segment (start 59.2682 66.3916) (end 55.9843 63.1077) (width 0.2) (layer "B.Cu") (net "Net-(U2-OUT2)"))
 (segment (start 59.9253 66.3916) (end 59.2682 66.3916) (width 0.2) (layer "B.Cu") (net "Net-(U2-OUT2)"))
 (segment (start 62.462 66.3428) (end 62.462 66.71) (width 0.2) (layer "B.Cu") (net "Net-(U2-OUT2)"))
 (segment (start 55.9843 62.2343) (end 54.5 60.75) (width 0.2) (layer "B.Cu") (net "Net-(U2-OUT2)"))
 (segment (start 65.0105 70.1042) (end 63.7647 71.35) (width 0.2) (layer "B.Cu") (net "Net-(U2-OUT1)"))
 (segment (start 55.2402 72.2098) (end 53.9995 72.2098) (width 0.2) (layer "B.Cu") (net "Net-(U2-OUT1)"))
 (segment (start 66.2658 70.1042) (end 65.0105 70.1042) (width 0.2) (layer "B.Cu") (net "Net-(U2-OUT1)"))
 (segment (start 53.3392 64.4108) (end 54.5 63.25) (width 0.2) (layer "B.Cu") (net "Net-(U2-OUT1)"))
 (segment (start 53.9995 72.2098) (end 53.3392 71.5495) (width 0.2) (layer "B.Cu") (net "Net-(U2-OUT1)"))
 (segment (start 63.7647 71.35) (end 56.1 71.35) (width 0.2) (layer "B.Cu") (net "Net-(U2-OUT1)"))
 (segment (start 56.1 71.35) (end 55.2402 72.2098) (width 0.2) (layer "B.Cu") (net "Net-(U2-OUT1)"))
 (segment (start 69.87 66.5) (end 66.2658 70.1042) (width 0.2) (layer "B.Cu") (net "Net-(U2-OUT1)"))
 (segment (start 53.3392 71.5495) (end 53.3392 64.4108) (width 0.2) (layer "B.Cu") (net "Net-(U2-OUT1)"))
 (segment (start 57.1283 71.1783) (end 65.5911 71.1783) (width 0.2) (layer "F.Cu") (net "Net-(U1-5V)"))
 (segment (start 65.5911 71.1783) (end 71.2629 65.5065) (width 0.2) (layer "F.Cu") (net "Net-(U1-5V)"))
 (segment (start 54.5 68.55) (end 57.1283 71.1783) (width 0.2) (layer "F.Cu") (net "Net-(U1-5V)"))
 (segment (start 65.5911 71.1783) (end 65.5911 71.1799) (width 0.2) (layer "F.Cu") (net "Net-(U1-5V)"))
 (segment (start 71.2629 65.5065) (end 71.2629 64.52) (width 0.2) (layer "F.Cu") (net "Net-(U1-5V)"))
 (segment (start 68.5861 60.4962) (end 62.9548 60.4962) (width 0.2) (layer "F.Cu") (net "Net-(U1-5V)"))
 (via (at 68.5861 60.4962) (size 0.6) (drill 0.3) (layers "F.Cu" "B.Cu") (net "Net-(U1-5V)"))
 (via (at 62.9548 60.4962) (size 0.6) (drill 0.3) (layers "F.Cu" "B.Cu") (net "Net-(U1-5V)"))
 (via (at 71.2629 64.52) (size 0.6) (drill 0.3) (layers "F.Cu" "B.Cu") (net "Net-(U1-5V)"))
 (via (at 65.5911 71.1799) (size 0.6) (drill 0.3) (layers "F.Cu" "B.Cu") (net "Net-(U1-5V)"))
 (segment (start 65.9169 71.7983) (end 66.75 71.7983) (width 0.2) (layer "B.Cu") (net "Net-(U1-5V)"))
 (segment (start 65.5 73.75) (end 64.7983 73.75) (width 0.2) (layer "B.Cu") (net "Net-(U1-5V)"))
 (segment (start 69.87 64.55) (end 71.0452 64.55) (width 0.2) (layer "B.Cu") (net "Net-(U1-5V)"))
 (segment (start 66.75 71.7082) (end 66.75 71.7983) (width 0.2) (layer "B.Cu") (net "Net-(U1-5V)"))
 (segment (start 75.7108 76.05) (end 75.7108 67.1187) (width 0.2) (layer "B.Cu") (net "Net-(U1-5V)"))
 (segment (start 69.573 71.0781) (end 67.3801 71.0781) (width 0.2) (layer "B.Cu") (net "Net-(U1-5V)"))
 (segment (start 69.2017 74.75) (end 70.6872 76.2355) (width 0.2) (layer "B.Cu") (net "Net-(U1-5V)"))
 (segment (start 69.87 64.55) (end 68.6948 64.55) (width 0.2) (layer "B.Cu") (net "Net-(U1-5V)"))
 (segment (start 68.7957 63.24) (end 68.6963 63.24) (width 0.2) (layer "B.Cu") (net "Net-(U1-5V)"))
 (segment (start 68.6963 63.24) (end 68.6948 63.24) (width 0.2) (layer "B.Cu") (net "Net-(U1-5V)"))
 (segment (start 65.5911 71.4725) (end 65.5911 71.1799) (width 0.2) (layer "B.Cu") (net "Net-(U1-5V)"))
 (segment (start 70.6872 76.2355) (end 75.5253 76.2355) (width 0.2) (layer "B.Cu") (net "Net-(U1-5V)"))
 (segment (start 80 76.05) (end 75.7108 76.05) (width 0.2) (layer "B.Cu") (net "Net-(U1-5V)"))
 (segment (start 68.5 74.75) (end 69.2017 74.75) (width 0.2) (layer "B.Cu") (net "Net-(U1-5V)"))
 (segment (start 64.7983 73.75) (end 64.7983 72.9169) (width 0.2) (layer "B.Cu") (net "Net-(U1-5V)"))
 (segment (start 68.6948 60.6049) (end 68.5861 60.4962) (width 0.2) (layer "B.Cu") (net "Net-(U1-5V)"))
 (segment (start 74.1668 66.4843) (end 69.573 71.0781) (width 0.2) (layer "B.Cu") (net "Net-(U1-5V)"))
 (segment (start 62.9548 61.94) (end 62.9548 60.4962) (width 0.2) (layer "B.Cu") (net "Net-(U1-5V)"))
 (segment (start 65.9169 71.7983) (end 65.5911 71.4725) (width 0.2) (layer "B.Cu") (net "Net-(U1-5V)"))
 (segment (start 68.6948 64.55) (end 68.6948 63.24) (width 0.2) (layer "B.Cu") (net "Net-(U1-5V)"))
 (segment (start 75.7108 67.1187) (end 75.0764 66.4843) (width 0.2) (layer "B.Cu") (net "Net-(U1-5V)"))
 (segment (start 66.75 72.5) (end 66.75 71.7983) (width 0.2) (layer "B.Cu") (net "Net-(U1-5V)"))
 (segment (start 67.3801 71.0781) (end 66.75 71.7082) (width 0.2) (layer "B.Cu") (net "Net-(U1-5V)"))
 (segment (start 75.0764 66.4843) (end 74.1668 66.4843) (width 0.2) (layer "B.Cu") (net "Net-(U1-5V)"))
 (segment (start 71.2629 64.52) (end 71.0752 64.52) (width 0.2) (layer "B.Cu") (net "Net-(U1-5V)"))
 (segment (start 75.5253 76.2355) (end 75.7108 76.05) (width 0.2) (layer "B.Cu") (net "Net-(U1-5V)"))
 (segment (start 69.87 63.24) (end 68.7957 63.24) (width 0.2) (layer "B.Cu") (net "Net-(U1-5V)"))
 (segment (start 68.6948 63.24) (end 68.6948 60.6049) (width 0.2) (layer "B.Cu") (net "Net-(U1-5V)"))
 (segment (start 71.0752 64.52) (end 71.0452 64.55) (width 0.2) (layer "B.Cu") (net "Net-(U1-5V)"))
 (segment (start 64.13 61.94) (end 62.9548 61.94) (width 0.2) (layer "B.Cu") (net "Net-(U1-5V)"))
 (segment (start 64.7983 72.9169) (end 65.9169 71.7983) (width 0.2) (layer "B.Cu") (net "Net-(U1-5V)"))
 (segment (start 81.19 69.86) (end 81.19 68.0934) (width 0.2) (layer "F.Cu") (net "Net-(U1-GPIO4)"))
 (segment (start 81.19 68.0934) (end 75.5566 62.46) (width 0.2) (layer "F.Cu") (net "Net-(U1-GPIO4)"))
 (segment (start 80 71.05) (end 81.19 69.86) (width 0.2) (layer "F.Cu") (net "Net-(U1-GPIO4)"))
 (segment (start 77.3399 73.7101) (end 54.6601 73.7101) (width 0.2) (layer "F.Cu") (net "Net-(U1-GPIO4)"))
 (segment (start 54.6601 73.7101) (end 54.5 73.55) (width 0.2) (layer "F.Cu") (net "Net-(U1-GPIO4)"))
 (segment (start 75.5566 62.46) (end 74.62 62.46) (width 0.2) (layer "F.Cu") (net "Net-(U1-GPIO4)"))
 (segment (start 80 71.05) (end 77.3399 73.7101) (width 0.2) (layer "F.Cu") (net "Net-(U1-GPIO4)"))
 (segment (start 70.9776 63.8953) (end 68.785 66.0879) (width 0.2) (layer "F.Cu") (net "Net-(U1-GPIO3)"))
 (segment (start 68.785 66.0879) (end 55.2421 66.0879) (width 0.2) (layer "F.Cu") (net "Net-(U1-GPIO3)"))
 (segment (start 53.3281 74.8781) (end 54.5 76.05) (width 0.2) (layer "F.Cu") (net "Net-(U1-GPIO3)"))
 (segment (start 55.2421 66.0879) (end 53.3281 68.0019) (width 0.2) (layer "F.Cu") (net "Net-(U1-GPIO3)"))
 (segment (start 80 68.55) (end 76.45 65) (width 0.2) (layer "F.Cu") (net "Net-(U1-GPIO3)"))
 (segment (start 53.3281 68.0019) (end 53.3281 74.8781) (width 0.2) (layer "F.Cu") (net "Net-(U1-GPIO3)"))
 (segment (start 74.62 65) (end 73.5153 63.8953) (width 0.2) (layer "F.Cu") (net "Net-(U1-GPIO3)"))
 (segment (start 76.45 65) (end 74.62 65) (width 0.2) (layer "F.Cu") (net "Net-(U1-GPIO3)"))
 (segment (start 73.5153 63.8953) (end 70.9776 63.8953) (width 0.2) (layer "F.Cu") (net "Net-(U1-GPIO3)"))
 (segment (start 68.5 73.25) (end 71.45 73.25) (width 0.2) (layer "B.Cu") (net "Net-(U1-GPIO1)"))
 (segment (start 71.45 73.25) (end 74.62 70.08) (width 0.2) (layer "B.Cu") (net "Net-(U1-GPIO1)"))
 (segment (start 67.25 72.5) (end 67.25 71.7983) (width 0.2) (layer "B.Cu") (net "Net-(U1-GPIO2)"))
 (segment (start 67.25 71.7983) (end 70.3617 71.7983) (width 0.2) (layer "B.Cu") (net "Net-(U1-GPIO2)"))
 (segment (start 70.3617 71.7983) (end 74.62 67.54) (width 0.2) (layer "B.Cu") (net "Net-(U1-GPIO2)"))
 (segment (start 71.9086 64.2708) (end 71.7085 64.0707) (width 0.2) (layer "B.Cu") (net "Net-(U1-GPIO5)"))
 (segment (start 71.7085 64.0707) (end 71.7085 61.1145) (width 0.2) (layer "B.Cu") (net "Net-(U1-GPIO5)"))
 (segment (start 72.5 65.14) (end 71.9086 65.14) (width 0.2) (layer "B.Cu") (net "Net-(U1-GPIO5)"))
 (segment (start 71.9086 65.14) (end 71.9086 64.2708) (width 0.2) (layer "B.Cu") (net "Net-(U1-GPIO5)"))
 (segment (start 71.9086 65.14) (end 71.1052 65.14) (width 0.2) (layer "B.Cu") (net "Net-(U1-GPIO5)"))
 (segment (start 71.1052 65.14) (end 71.0452 65.2) (width 0.2) (layer "B.Cu") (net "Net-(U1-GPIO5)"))
 (segment (start 71.7085 61.1145) (end 72.903 59.92) (width 0.2) (layer "B.Cu") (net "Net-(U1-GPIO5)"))
 (segment (start 69.87 65.2) (end 71.0452 65.2) (width 0.2) (layer "B.Cu") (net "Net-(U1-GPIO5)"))
 (segment (start 72.903 59.92) (end 74.62 59.92) (width 0.2) (layer "B.Cu") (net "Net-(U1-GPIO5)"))
 (segment (start 69.87 63.9) (end 71.0452 63.9) (width 0.2) (layer "B.Cu") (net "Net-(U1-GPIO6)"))
 (segment (start 71.0452 60.9548) (end 74.62 57.38) (width 0.2) (layer "B.Cu") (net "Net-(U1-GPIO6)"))
 (segment (start 71.0452 63.9) (end 71.0452 60.9548) (width 0.2) (layer "B.Cu") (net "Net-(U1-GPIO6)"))
 (segment (start 62.92 63.24) (end 61.5 61.82) (width 0.2) (layer "B.Cu") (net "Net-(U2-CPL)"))
 (segment (start 64.13 63.24) (end 62.92 63.24) (width 0.2) (layer "B.Cu") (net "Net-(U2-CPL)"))
 (segment (start 62.9317 63.9) (end 62.2517 63.22) (width 0.2) (layer "B.Cu") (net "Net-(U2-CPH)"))
 (segment (start 64.13 63.9) (end 62.9317 63.9) (width 0.2) (layer "B.Cu") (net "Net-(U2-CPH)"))
 (segment (start 61.5 63.22) (end 62.2517 63.22) (width 0.2) (layer "B.Cu") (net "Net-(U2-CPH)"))
 (segment (start 64.13 64.55) (end 62.9217 64.55) (width 0.2) (layer "B.Cu") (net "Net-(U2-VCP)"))
 (segment (start 62.9217 64.55) (end 62.2517 65.22) (width 0.2) (layer "B.Cu") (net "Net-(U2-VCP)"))
 (segment (start 61.5 65.22) (end 62.2517 65.22) (width 0.2) (layer "B.Cu") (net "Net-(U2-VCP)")))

